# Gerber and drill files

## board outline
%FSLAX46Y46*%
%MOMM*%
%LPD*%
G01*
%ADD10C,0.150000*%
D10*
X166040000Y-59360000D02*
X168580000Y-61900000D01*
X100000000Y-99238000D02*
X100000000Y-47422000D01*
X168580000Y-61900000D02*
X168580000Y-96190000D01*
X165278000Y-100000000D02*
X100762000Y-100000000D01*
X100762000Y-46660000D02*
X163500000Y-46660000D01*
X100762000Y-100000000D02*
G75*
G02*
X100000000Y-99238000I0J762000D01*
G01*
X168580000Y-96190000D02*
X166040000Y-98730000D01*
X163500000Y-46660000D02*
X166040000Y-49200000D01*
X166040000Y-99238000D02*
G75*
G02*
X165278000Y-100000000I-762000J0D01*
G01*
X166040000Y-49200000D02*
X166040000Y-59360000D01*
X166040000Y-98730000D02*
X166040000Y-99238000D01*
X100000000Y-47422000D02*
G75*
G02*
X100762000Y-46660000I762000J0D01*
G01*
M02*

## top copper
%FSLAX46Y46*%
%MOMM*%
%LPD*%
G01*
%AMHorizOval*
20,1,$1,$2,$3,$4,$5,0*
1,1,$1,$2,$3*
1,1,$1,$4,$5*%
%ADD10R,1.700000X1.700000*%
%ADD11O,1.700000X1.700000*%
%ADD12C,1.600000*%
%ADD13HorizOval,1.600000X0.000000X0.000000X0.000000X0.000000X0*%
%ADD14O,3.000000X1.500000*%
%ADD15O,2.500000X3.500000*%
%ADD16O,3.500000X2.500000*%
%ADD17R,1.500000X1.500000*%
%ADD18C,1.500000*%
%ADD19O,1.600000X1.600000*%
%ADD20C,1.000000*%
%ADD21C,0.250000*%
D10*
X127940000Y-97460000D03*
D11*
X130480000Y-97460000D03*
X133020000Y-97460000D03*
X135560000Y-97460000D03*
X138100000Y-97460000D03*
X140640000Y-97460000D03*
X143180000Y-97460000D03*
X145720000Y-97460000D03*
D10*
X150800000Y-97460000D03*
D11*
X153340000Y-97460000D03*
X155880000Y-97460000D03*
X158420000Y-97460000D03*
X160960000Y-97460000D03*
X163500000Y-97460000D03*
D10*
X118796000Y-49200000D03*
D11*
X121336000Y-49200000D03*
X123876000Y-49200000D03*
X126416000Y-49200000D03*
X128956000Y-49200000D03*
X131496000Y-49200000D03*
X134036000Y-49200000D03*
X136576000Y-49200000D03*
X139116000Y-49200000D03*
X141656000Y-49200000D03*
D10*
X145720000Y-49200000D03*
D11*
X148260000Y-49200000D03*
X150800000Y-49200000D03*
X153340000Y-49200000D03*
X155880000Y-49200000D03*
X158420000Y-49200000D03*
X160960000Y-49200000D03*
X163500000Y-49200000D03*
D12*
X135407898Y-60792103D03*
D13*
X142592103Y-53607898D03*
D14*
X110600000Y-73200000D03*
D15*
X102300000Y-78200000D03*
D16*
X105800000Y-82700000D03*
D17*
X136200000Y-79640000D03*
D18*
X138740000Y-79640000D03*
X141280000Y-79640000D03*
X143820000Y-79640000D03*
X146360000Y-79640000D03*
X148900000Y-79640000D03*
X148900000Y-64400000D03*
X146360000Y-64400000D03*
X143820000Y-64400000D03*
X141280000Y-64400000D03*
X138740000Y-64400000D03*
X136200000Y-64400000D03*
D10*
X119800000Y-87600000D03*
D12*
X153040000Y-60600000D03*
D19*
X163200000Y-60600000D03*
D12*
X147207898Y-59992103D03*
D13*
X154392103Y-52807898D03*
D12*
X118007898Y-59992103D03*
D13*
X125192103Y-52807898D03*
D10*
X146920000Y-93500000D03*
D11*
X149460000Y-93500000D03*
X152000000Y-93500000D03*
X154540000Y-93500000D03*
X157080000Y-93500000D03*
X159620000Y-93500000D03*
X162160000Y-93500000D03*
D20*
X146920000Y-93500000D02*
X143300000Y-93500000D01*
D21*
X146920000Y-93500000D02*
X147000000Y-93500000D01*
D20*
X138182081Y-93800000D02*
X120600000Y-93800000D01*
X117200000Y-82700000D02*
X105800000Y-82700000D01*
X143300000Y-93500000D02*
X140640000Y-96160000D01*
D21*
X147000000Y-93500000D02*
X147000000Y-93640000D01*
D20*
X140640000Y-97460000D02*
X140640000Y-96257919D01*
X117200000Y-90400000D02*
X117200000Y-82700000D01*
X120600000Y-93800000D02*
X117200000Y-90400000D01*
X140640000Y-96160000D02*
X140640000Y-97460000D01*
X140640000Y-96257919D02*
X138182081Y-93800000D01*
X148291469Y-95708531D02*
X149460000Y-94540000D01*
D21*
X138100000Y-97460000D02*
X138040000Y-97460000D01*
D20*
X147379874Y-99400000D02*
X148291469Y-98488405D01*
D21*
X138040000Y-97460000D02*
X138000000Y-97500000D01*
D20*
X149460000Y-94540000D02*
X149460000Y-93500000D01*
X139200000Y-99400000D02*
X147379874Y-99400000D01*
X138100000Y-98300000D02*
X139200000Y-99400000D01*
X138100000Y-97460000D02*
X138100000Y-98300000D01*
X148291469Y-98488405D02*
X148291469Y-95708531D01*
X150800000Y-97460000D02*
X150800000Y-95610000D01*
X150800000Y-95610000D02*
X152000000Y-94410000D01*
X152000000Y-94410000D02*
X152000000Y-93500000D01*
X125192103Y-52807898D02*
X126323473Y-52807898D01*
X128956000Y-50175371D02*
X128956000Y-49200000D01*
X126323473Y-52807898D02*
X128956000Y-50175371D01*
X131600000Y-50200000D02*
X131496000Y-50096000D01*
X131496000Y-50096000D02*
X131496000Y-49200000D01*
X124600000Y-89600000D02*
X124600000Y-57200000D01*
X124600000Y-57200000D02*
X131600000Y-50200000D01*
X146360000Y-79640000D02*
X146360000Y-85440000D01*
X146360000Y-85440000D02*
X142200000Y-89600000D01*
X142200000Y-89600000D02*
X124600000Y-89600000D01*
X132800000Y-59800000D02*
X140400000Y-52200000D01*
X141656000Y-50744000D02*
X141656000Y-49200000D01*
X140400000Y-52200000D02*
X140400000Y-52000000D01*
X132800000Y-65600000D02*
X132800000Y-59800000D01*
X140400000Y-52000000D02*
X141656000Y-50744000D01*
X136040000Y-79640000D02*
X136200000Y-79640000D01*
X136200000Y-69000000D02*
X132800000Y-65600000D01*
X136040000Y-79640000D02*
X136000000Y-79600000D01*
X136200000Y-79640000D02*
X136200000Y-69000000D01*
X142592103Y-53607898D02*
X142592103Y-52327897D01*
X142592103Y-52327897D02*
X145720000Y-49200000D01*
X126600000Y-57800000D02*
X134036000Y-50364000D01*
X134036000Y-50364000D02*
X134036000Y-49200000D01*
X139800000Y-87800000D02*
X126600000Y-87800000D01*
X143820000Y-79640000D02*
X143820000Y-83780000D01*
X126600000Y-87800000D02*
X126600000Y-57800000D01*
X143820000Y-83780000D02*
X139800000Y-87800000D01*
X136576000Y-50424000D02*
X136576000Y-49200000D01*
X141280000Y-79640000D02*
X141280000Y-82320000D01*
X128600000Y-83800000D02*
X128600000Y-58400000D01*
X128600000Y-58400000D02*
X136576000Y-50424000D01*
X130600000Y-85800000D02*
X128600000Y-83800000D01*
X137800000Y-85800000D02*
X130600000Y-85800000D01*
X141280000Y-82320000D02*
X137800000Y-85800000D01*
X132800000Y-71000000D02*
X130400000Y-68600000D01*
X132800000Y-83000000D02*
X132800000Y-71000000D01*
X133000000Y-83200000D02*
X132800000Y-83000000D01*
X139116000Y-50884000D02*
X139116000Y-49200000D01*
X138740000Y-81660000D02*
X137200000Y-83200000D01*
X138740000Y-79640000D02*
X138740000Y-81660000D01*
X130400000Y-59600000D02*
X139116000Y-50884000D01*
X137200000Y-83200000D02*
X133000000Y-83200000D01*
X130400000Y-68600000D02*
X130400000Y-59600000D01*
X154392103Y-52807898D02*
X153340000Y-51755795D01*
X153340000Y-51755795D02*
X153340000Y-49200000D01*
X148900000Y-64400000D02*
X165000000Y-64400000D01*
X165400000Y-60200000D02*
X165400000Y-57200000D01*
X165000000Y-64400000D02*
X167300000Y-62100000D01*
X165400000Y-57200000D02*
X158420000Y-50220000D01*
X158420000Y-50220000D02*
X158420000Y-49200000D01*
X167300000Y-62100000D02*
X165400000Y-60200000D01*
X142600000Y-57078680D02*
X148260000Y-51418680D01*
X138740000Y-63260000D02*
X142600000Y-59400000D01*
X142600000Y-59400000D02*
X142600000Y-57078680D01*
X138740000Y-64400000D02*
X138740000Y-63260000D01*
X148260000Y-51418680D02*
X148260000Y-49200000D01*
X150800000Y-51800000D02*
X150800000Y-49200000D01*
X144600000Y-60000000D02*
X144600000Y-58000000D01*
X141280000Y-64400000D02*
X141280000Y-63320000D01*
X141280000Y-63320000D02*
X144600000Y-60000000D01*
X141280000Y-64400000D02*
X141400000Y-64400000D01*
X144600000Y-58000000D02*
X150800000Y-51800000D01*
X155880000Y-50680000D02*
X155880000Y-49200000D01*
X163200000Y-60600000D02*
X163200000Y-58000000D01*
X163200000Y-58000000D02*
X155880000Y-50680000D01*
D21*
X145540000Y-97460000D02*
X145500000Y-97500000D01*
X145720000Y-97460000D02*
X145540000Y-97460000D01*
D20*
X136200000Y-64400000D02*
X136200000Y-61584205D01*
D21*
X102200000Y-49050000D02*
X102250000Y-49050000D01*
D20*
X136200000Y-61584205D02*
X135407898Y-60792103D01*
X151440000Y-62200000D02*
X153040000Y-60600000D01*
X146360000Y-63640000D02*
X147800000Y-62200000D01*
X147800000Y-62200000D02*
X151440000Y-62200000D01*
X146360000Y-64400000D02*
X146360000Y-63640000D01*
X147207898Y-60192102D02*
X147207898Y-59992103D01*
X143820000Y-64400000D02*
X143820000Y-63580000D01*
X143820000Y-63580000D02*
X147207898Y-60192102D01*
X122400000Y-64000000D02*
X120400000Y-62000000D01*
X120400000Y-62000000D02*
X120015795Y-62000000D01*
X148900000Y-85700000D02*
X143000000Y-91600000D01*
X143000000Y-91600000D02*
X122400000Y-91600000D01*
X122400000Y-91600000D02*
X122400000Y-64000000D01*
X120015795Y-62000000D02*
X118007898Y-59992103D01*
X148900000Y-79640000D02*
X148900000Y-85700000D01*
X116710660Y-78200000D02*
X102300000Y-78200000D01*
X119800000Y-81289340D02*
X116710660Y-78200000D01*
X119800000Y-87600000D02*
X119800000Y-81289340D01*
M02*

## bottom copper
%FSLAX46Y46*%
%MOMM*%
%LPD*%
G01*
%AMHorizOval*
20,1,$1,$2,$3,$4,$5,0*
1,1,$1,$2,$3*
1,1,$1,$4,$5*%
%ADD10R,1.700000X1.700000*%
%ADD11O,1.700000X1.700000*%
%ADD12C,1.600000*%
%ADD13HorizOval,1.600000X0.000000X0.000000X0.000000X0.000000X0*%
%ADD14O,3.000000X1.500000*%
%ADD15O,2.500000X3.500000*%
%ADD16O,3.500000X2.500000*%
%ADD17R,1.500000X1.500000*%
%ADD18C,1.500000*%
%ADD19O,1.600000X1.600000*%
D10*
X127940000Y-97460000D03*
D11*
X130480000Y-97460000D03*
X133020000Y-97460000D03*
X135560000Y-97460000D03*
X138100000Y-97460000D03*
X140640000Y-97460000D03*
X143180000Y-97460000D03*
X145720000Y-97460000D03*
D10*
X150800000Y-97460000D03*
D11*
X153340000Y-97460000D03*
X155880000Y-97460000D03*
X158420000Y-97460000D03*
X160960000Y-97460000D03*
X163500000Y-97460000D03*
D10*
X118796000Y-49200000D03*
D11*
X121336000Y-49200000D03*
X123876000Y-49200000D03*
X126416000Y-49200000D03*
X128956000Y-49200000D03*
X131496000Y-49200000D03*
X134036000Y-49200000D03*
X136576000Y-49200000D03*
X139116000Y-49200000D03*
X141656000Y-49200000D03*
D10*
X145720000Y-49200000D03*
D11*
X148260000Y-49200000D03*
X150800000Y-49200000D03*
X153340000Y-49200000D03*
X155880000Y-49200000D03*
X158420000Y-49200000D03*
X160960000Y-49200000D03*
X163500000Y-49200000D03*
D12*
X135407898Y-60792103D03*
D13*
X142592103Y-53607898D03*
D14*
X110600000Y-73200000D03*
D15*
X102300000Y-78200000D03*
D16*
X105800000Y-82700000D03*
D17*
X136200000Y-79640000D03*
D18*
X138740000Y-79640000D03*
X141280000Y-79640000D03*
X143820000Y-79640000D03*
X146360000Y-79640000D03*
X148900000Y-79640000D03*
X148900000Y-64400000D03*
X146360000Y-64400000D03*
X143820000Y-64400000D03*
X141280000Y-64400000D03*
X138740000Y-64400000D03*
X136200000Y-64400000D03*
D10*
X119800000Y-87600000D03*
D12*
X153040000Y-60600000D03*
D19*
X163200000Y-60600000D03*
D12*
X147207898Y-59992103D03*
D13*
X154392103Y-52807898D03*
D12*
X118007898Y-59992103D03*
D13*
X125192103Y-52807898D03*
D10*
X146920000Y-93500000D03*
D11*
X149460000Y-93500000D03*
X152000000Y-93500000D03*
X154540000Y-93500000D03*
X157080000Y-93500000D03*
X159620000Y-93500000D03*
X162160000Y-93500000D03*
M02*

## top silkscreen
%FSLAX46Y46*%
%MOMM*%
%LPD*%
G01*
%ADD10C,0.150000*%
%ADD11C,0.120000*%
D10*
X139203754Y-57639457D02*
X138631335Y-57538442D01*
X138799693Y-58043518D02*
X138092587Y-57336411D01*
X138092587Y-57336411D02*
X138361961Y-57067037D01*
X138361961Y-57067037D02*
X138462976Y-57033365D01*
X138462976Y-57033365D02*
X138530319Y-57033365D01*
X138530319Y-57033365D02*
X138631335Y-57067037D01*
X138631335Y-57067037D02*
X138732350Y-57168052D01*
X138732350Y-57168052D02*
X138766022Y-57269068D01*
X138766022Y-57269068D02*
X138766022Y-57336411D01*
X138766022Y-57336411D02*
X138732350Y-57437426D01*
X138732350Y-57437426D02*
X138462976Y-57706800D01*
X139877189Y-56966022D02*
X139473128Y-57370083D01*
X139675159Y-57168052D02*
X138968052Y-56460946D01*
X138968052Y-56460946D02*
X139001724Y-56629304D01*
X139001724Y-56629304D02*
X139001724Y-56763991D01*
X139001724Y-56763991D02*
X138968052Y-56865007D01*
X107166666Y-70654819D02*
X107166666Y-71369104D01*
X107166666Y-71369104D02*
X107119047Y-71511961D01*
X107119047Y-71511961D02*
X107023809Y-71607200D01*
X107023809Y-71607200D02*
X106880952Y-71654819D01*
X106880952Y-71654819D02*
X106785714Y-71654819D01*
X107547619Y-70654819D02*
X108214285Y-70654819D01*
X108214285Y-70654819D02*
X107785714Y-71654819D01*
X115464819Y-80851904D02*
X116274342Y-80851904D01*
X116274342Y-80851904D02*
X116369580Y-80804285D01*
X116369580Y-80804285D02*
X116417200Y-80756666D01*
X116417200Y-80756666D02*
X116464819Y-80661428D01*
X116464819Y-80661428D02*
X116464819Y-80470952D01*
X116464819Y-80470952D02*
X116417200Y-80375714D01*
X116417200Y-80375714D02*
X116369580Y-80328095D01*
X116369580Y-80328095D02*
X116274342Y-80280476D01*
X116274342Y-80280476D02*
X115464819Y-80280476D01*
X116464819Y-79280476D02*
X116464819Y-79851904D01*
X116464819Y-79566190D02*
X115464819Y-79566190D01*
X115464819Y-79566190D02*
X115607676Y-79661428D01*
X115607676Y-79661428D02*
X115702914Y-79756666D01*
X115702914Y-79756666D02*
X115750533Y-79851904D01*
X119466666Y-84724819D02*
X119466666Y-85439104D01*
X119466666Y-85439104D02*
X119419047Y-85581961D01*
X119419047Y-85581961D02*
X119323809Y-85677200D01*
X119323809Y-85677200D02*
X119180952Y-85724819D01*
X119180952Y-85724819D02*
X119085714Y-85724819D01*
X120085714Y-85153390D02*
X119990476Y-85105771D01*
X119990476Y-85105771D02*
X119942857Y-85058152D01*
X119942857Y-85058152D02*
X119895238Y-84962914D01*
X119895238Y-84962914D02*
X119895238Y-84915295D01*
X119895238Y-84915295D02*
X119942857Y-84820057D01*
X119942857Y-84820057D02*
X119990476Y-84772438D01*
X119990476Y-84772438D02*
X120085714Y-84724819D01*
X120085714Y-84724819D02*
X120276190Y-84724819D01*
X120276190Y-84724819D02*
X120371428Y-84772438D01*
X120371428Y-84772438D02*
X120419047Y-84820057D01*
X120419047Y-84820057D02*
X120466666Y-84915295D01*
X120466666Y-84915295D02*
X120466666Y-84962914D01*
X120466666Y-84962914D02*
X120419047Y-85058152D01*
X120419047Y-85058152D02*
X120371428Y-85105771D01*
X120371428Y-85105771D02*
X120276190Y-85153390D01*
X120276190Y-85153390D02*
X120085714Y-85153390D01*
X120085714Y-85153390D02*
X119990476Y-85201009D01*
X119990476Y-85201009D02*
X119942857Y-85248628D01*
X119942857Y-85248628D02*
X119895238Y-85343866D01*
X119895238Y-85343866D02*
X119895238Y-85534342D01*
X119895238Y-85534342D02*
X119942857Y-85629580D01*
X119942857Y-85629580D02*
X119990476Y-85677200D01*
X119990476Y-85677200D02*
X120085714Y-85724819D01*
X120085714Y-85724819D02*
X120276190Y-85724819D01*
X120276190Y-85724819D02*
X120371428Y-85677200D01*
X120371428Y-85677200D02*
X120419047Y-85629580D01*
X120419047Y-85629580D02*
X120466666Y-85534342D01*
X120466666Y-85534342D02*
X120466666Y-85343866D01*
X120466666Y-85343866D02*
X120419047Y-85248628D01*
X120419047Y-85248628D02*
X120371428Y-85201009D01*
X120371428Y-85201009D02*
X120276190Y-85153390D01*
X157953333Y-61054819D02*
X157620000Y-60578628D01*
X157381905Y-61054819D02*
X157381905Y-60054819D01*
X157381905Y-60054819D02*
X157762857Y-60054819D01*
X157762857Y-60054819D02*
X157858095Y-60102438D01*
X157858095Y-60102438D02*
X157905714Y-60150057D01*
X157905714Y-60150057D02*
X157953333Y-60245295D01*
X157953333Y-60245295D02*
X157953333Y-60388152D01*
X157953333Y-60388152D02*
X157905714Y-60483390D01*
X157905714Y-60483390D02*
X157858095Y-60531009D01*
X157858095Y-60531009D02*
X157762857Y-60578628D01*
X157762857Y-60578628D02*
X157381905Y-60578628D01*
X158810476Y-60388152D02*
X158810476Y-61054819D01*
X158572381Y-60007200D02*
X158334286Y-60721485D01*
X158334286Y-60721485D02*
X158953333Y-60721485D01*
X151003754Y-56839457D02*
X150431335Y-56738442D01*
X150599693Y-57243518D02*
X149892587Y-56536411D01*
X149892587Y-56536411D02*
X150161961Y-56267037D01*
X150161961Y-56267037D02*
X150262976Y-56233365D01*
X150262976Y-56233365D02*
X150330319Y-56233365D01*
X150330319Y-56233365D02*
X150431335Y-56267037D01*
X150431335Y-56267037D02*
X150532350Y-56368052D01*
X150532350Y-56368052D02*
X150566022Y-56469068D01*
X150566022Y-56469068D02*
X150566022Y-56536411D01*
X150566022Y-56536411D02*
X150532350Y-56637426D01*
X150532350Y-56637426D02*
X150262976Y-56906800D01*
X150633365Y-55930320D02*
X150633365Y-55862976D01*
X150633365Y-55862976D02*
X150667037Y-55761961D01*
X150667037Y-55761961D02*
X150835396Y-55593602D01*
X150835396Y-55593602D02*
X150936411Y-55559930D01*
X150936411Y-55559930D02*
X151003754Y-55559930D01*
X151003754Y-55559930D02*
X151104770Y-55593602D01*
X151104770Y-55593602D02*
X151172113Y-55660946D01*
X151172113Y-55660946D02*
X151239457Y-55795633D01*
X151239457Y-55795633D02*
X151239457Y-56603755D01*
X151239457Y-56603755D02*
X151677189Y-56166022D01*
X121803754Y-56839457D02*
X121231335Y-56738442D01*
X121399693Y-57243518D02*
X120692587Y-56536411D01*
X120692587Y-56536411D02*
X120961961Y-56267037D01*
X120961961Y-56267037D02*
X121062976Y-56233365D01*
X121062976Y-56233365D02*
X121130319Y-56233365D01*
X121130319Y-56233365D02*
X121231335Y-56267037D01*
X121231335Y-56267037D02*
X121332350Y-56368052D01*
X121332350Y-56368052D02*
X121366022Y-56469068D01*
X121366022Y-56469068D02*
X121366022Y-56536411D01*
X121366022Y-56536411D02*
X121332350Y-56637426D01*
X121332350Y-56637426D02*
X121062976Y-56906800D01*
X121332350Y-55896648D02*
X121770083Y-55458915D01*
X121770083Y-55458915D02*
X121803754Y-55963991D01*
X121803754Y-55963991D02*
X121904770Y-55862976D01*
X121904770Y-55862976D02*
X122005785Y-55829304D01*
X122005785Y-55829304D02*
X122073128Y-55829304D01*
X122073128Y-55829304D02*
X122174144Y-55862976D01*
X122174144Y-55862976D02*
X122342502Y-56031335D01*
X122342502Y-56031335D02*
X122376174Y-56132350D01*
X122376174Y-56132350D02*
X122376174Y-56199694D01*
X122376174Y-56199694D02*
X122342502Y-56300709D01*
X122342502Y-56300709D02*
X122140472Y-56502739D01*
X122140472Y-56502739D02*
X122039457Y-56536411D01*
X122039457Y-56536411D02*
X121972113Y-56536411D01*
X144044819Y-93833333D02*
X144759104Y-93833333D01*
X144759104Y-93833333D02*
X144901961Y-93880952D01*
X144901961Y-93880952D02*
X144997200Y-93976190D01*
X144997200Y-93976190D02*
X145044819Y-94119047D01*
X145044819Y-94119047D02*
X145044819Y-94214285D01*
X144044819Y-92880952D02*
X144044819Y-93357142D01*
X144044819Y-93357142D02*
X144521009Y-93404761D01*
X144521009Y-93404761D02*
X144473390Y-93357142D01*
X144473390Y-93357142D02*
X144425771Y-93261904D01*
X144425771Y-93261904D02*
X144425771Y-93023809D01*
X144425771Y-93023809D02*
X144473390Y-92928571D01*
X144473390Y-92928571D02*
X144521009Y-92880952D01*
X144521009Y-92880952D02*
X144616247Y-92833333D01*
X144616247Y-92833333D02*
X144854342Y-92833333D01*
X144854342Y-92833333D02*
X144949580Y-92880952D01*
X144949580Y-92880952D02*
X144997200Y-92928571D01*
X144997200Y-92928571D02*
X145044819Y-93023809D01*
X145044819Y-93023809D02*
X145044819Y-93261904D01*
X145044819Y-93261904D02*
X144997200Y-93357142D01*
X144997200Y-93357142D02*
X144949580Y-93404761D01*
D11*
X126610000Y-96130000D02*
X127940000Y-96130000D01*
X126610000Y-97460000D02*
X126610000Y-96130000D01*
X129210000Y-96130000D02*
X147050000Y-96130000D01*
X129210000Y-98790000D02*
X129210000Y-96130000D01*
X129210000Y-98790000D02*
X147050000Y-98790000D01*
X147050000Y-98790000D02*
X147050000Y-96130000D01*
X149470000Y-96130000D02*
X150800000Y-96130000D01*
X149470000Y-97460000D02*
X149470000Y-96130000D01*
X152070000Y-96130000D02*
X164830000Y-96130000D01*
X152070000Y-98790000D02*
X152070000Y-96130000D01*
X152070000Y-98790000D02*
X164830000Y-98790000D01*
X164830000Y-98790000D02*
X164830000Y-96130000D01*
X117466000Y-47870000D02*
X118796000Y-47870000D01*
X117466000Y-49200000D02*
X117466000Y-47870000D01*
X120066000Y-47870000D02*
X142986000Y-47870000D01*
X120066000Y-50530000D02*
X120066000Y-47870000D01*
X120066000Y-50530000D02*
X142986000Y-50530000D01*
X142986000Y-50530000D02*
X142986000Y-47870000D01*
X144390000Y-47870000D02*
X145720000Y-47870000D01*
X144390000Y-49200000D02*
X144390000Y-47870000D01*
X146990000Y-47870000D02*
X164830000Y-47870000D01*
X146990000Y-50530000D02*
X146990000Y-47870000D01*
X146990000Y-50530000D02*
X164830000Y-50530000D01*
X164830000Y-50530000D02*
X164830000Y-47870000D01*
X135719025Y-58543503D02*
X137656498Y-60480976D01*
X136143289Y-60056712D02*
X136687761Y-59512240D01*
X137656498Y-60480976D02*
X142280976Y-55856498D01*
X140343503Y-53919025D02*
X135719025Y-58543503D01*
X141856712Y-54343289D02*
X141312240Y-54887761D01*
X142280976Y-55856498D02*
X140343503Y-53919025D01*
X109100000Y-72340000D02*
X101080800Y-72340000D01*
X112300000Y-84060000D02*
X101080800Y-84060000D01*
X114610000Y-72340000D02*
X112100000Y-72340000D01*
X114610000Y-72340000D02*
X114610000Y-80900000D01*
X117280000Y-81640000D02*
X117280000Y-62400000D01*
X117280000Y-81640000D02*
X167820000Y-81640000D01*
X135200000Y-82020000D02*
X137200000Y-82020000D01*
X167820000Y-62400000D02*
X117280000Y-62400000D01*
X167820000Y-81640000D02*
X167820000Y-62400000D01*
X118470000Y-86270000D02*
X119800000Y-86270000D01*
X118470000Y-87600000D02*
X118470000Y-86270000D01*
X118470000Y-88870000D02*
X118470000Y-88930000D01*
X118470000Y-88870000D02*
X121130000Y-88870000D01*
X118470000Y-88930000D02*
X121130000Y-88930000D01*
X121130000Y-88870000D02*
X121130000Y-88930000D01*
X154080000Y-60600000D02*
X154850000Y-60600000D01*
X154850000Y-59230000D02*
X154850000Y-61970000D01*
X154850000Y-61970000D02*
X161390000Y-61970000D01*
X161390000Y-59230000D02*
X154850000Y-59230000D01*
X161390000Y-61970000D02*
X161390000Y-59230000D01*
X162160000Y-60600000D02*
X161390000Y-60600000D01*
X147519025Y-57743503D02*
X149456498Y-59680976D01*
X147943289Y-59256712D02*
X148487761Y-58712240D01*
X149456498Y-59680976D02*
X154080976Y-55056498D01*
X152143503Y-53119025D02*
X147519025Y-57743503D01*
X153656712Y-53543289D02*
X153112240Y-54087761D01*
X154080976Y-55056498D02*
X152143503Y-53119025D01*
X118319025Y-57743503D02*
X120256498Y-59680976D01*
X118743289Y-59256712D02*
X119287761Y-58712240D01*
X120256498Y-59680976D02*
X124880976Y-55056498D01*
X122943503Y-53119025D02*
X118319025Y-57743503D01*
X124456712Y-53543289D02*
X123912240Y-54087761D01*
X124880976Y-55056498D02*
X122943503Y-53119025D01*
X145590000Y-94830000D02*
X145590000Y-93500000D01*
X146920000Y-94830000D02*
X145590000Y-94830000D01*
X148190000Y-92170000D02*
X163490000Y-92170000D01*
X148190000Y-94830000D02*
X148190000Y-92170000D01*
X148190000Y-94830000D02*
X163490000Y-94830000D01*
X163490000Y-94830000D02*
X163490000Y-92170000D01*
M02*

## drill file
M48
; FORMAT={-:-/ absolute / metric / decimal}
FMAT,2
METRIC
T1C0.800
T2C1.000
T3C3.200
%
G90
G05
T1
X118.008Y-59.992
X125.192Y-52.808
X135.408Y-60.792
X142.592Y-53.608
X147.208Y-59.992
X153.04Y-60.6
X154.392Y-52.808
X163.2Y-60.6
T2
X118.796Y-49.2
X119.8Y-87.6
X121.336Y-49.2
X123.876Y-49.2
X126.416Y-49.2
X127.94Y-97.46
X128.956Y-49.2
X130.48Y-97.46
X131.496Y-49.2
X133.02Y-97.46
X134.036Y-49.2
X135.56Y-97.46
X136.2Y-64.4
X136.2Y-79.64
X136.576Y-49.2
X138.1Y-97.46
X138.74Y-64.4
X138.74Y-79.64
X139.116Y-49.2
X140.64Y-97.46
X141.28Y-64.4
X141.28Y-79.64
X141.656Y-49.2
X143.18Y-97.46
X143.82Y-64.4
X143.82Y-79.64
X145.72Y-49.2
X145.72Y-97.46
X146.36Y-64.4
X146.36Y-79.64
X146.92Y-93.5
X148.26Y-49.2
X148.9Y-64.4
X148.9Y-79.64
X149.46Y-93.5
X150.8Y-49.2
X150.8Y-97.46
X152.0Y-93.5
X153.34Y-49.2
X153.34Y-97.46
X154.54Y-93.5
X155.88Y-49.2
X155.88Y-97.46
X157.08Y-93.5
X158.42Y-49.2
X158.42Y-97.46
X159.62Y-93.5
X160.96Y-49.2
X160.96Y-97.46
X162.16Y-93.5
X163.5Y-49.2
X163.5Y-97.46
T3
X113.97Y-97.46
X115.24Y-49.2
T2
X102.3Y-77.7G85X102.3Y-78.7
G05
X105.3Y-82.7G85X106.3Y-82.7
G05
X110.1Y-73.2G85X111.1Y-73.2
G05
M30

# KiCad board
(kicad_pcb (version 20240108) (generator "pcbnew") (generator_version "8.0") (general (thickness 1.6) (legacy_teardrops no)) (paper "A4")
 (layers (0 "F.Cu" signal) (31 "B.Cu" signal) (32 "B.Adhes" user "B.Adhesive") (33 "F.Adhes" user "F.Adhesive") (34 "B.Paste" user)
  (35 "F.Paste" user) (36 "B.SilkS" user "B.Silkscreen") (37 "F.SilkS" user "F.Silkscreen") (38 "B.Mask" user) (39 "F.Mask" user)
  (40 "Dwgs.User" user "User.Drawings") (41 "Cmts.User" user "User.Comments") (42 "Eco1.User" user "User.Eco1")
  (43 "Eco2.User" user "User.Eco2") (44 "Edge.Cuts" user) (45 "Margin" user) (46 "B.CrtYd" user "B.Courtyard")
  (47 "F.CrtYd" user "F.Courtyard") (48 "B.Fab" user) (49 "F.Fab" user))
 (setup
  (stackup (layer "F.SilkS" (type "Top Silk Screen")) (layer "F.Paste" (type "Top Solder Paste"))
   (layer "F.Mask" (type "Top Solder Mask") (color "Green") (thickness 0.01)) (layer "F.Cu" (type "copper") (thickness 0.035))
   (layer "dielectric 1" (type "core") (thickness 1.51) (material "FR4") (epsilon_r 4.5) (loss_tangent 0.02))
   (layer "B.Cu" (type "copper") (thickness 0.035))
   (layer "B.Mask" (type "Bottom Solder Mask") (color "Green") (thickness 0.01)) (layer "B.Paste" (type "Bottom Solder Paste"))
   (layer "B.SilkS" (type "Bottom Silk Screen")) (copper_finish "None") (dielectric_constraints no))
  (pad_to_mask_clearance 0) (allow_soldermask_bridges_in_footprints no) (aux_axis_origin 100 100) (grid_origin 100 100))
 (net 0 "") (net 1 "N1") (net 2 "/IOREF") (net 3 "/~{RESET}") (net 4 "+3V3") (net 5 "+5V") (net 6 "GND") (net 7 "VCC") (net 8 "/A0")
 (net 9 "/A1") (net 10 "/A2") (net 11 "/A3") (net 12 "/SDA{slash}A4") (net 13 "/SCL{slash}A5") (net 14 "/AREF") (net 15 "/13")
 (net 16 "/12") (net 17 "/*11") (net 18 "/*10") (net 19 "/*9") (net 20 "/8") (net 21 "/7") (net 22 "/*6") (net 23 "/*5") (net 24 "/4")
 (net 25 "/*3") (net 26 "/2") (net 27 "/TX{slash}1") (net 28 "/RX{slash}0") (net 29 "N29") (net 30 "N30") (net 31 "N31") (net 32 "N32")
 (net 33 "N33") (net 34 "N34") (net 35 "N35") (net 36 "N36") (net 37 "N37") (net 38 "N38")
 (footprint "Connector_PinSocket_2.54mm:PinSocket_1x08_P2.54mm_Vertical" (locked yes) (layer "F.Cu") (at 127.94 97.46 90)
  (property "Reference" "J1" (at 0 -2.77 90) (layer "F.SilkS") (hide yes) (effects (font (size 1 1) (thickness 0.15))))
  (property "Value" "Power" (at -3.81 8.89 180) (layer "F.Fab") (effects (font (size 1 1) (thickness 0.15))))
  (fp_line (start 1.33 -1.33) (end 1.33 0) (stroke (width 0.12) (type solid)) (layer "F.SilkS"))
  (fp_line (start 0 -1.33) (end 1.33 -1.33) (stroke (width 0.12) (type solid)) (layer "F.SilkS"))
  (fp_line (start 1.33 1.27) (end 1.33 19.11) (stroke (width 0.12) (type solid)) (layer "F.SilkS"))
  (fp_line (start -1.33 1.27) (end 1.33 1.27) (stroke (width 0.12) (type solid)) (layer "F.SilkS"))
  (fp_line (start -1.33 1.27) (end -1.33 19.11) (stroke (width 0.12) (type solid)) (layer "F.SilkS"))
  (fp_line (start -1.33 19.11) (end 1.33 19.11) (stroke (width 0.12) (type solid)) (layer "F.SilkS"))
  (pad "1" thru_hole rect (at 0 0 90) (size 1.7 1.7) (drill 1) (layers "*.Cu" "*.Mask") (remove_unused_layers no) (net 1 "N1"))
  (pad "2" thru_hole oval (at 0 2.54 90) (size 1.7 1.7) (drill 1) (layers "*.Cu" "*.Mask") (remove_unused_layers no) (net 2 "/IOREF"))
  (pad "3" thru_hole oval (at 0 5.08 90) (size 1.7 1.7) (drill 1) (layers "*.Cu" "*.Mask") (remove_unused_layers no) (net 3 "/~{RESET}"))
  (pad "4" thru_hole oval (at 0 7.62 90) (size 1.7 1.7) (drill 1) (layers "*.Cu" "*.Mask") (remove_unused_layers no) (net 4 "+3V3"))
  (pad "5" thru_hole oval (at 0 10.16 90) (size 1.7 1.7) (drill 1) (layers "*.Cu" "*.Mask") (remove_unused_layers no) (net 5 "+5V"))
  (pad "6" thru_hole oval (at 0 12.7 90) (size 1.7 1.7) (drill 1) (layers "*.Cu" "*.Mask") (remove_unused_layers no) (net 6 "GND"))
  (pad "7" thru_hole oval (at 0 15.24 90) (size 1.7 1.7) (drill 1) (layers "*.Cu" "*.Mask") (remove_unused_layers no) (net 6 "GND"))
  (pad "8" thru_hole oval (at 0 17.78 90) (size 1.7 1.7) (drill 1) (layers "*.Cu" "*.Mask") (remove_unused_layers no) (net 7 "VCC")))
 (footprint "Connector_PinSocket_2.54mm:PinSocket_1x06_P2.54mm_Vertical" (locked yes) (layer "F.Cu") (at 150.8 97.46 90)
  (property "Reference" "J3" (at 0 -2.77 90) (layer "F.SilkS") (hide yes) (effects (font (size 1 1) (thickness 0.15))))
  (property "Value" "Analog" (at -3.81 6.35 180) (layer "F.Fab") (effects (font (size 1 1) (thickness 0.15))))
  (fp_line (start 1.33 -1.33) (end 1.33 0) (stroke (width 0.12) (type solid)) (layer "F.SilkS"))
  (fp_line (start 0 -1.33) (end 1.33 -1.33) (stroke (width 0.12) (type solid)) (layer "F.SilkS"))
  (fp_line (start 1.33 1.27) (end 1.33 14.03) (stroke (width 0.12) (type solid)) (layer "F.SilkS"))
  (fp_line (start -1.33 1.27) (end 1.33 1.27) (stroke (width 0.12) (type solid)) (layer "F.SilkS"))
  (fp_line (start -1.33 1.27) (end -1.33 14.03) (stroke (width 0.12) (type solid)) (layer "F.SilkS"))
  (fp_line (start -1.33 14.03) (end 1.33 14.03) (stroke (width 0.12) (type solid)) (layer "F.SilkS"))
  (pad "1" thru_hole rect (at 0 0 90) (size 1.7 1.7) (drill 1) (layers "*.Cu" "*.Mask") (remove_unused_layers no) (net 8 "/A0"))
  (pad "2" thru_hole oval (at 0 2.54 90) (size 1.7 1.7) (drill 1) (layers "*.Cu" "*.Mask") (remove_unused_layers no) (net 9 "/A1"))
  (pad "3" thru_hole oval (at 0 5.08 90) (size 1.7 1.7) (drill 1) (layers "*.Cu" "*.Mask") (remove_unused_layers no) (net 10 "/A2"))
  (pad "4" thru_hole oval (at 0 7.62 90) (size 1.7 1.7) (drill 1) (layers "*.Cu" "*.Mask") (remove_unused_layers no) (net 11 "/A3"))
  (pad "5" thru_hole oval (at 0 10.16 90) (size 1.7 1.7) (drill 1) (layers "*.Cu" "*.Mask") (remove_unused_layers no)
   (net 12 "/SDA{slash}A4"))
  (pad "6" thru_hole oval (at 0 12.7 90) (size 1.7 1.7) (drill 1) (layers "*.Cu" "*.Mask") (remove_unused_layers no)
   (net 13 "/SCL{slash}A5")))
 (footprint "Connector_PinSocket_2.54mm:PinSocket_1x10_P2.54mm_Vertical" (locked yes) (layer "F.Cu") (at 118.796 49.2 90)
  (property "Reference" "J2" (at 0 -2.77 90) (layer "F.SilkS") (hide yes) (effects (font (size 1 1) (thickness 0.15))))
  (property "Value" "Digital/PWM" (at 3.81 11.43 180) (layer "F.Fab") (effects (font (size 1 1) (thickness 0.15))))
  (fp_line (start 1.33 -1.33) (end 1.33 0) (stroke (width 0.12) (type solid)) (layer "F.SilkS"))
  (fp_line (start 0 -1.33) (end 1.33 -1.33) (stroke (width 0.12) (type solid)) (layer "F.SilkS"))
  (fp_line (start 1.33 1.27) (end 1.33 24.19) (stroke (width 0.12) (type solid)) (layer "F.SilkS"))
  (fp_line (start -1.33 1.27) (end 1.33 1.27) (stroke (width 0.12) (type solid)) (layer "F.SilkS"))
  (fp_line (start -1.33 1.27) (end -1.33 24.19) (stroke (width 0.12) (type solid)) (layer "F.SilkS"))
  (fp_line (start -1.33 24.19) (end 1.33 24.19) (stroke (width 0.12) (type solid)) (layer "F.SilkS"))
  (pad "1" thru_hole rect (at 0 0 90) (size 1.7 1.7) (drill 1) (layers "*.Cu" "*.Mask") (remove_unused_layers no) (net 13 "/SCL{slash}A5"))
  (pad "2" thru_hole oval (at 0 2.54 90) (size 1.7 1.7) (drill 1) (layers "*.Cu" "*.Mask") (remove_unused_layers no)
   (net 12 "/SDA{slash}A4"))
  (pad "3" thru_hole oval (at 0 5.08 90) (size 1.7 1.7) (drill 1) (layers "*.Cu" "*.Mask") (remove_unused_layers no) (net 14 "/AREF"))
  (pad "4" thru_hole oval (at 0 7.62 90) (size 1.7 1.7) (drill 1) (layers "*.Cu" "*.Mask") (remove_unused_layers no) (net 6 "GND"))
  (pad "5" thru_hole oval (at 0 10.16 90) (size 1.7 1.7) (drill 1) (layers "*.Cu" "*.Mask") (remove_unused_layers no) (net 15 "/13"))
  (pad "6" thru_hole oval (at 0 12.7 90) (size 1.7 1.7) (drill 1) (layers "*.Cu" "*.Mask") (remove_unused_layers no) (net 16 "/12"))
  (pad "7" thru_hole oval (at 0 15.24 90) (size 1.7 1.7) (drill 1) (layers "*.Cu" "*.Mask") (remove_unused_layers no) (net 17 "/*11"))
  (pad "8" thru_hole oval (at 0 17.78 90) (size 1.7 1.7) (drill 1) (layers "*.Cu" "*.Mask") (remove_unused_layers no) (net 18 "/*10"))
  (pad "9" thru_hole oval (at 0 20.32 90) (size 1.7 1.7) (drill 1) (layers "*.Cu" "*.Mask") (remove_unused_layers no) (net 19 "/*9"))
  (pad "10" thru_hole oval (at 0 22.86 90) (size 1.7 1.7) (drill 1) (layers "*.Cu" "*.Mask") (remove_unused_layers no) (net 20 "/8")))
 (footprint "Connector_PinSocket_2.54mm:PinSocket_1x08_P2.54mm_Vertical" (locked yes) (layer "F.Cu") (at 145.72 49.2 90)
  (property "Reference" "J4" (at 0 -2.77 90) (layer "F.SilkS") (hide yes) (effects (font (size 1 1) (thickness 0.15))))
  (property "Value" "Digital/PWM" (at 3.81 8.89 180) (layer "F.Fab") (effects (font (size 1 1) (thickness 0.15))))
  (fp_line (start 1.33 -1.33) (end 1.33 0) (stroke (width 0.12) (type solid)) (layer "F.SilkS"))
  (fp_line (start 0 -1.33) (end 1.33 -1.33) (stroke (width 0.12) (type solid)) (layer "F.SilkS"))
  (fp_line (start 1.33 1.27) (end 1.33 19.11) (stroke (width 0.12) (type solid)) (layer "F.SilkS"))
  (fp_line (start -1.33 1.27) (end 1.33 1.27) (stroke (width 0.12) (type solid)) (layer "F.SilkS"))
  (fp_line (start -1.33 1.27) (end -1.33 19.11) (stroke (width 0.12) (type solid)) (layer "F.SilkS"))
  (fp_line (start -1.33 19.11) (end 1.33 19.11) (stroke (width 0.12) (type solid)) (layer "F.SilkS"))
  (pad "1" thru_hole rect (at 0 0 90) (size 1.7 1.7) (drill 1) (layers "*.Cu" "*.Mask") (remove_unused_layers no) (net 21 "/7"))
  (pad "2" thru_hole oval (at 0 2.54 90) (size 1.7 1.7) (drill 1) (layers "*.Cu" "*.Mask") (remove_unused_layers no) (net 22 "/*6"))
  (pad "3" thru_hole oval (at 0 5.08 90) (size 1.7 1.7) (drill 1) (layers "*.Cu" "*.Mask") (remove_unused_layers no) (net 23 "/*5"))
  (pad "4" thru_hole oval (at 0 7.62 90) (size 1.7 1.7) (drill 1) (layers "*.Cu" "*.Mask") (remove_unused_layers no) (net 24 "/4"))
  (pad "5" thru_hole oval (at 0 10.16 90) (size 1.7 1.7) (drill 1) (layers "*.Cu" "*.Mask") (remove_unused_layers no) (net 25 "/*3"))
  (pad "6" thru_hole oval (at 0 12.7 90) (size 1.7 1.7) (drill 1) (layers "*.Cu" "*.Mask") (remove_unused_layers no) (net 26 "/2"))
  (pad "7" thru_hole oval (at 0 15.24 90) (size 1.7 1.7) (drill 1) (layers "*.Cu" "*.Mask") (remove_unused_layers no) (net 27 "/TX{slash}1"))
  (pad "8" thru_hole oval (at 0 17.78 90) (size 1.7 1.7) (drill 1) (layers "*.Cu" "*.Mask") (remove_unused_layers no) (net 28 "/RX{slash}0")))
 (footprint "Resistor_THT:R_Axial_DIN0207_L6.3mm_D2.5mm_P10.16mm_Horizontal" (layer "F.Cu") (at 135.407898 60.792103 45)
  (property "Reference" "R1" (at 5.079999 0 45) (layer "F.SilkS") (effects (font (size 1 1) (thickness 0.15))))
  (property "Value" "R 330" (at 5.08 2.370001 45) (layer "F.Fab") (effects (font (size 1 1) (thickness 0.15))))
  (fp_line (start 1.81 -1.37) (end 1.81 1.37) (stroke (width 0.12) (type solid)) (layer "F.SilkS"))
  (fp_line (start 1.04 0) (end 1.81 0) (stroke (width 0.12) (type solid)) (layer "F.SilkS"))
  (fp_line (start 1.81 1.37) (end 8.35 1.37) (stroke (width 0.12) (type solid)) (layer "F.SilkS"))
  (fp_line (start 8.35 -1.37) (end 1.81 -1.37) (stroke (width 0.12) (type solid)) (layer "F.SilkS"))
  (fp_line (start 9.12 0) (end 8.350001 0) (stroke (width 0.12) (type solid)) (layer "F.SilkS"))
  (fp_line (start 8.35 1.37) (end 8.35 -1.37) (stroke (width 0.12) (type solid)) (layer "F.SilkS"))
  (pad "1" thru_hole circle (at 0 0 45) (size 1.6 1.6) (drill 0.8) (layers "*.Cu" "*.Mask") (remove_unused_layers no) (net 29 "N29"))
  (pad "2" thru_hole oval (at 10.16 0 45) (size 1.6 1.6) (drill 0.8) (layers "*.Cu" "*.Mask") (remove_unused_layers no) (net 21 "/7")))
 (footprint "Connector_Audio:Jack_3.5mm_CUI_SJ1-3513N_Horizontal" (layer "F.Cu") (at 102.3 78.2)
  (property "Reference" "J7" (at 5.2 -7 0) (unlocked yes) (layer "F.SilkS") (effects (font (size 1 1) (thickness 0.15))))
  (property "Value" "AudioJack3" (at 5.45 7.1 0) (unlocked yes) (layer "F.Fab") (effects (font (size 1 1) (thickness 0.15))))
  (fp_line (start 6.8 -5.86) (end -1.2192 -5.86) (stroke (width 0.12) (type solid)) (layer "F.SilkS"))
  (fp_line (start 10 5.86) (end -1.2192 5.86) (stroke (width 0.12) (type solid)) (layer "F.SilkS"))
  (fp_line (start 12.31 -5.86) (end 9.8 -5.86) (stroke (width 0.12) (type solid)) (layer "F.SilkS"))
  (fp_line (start 12.31 -5.86) (end 12.31 2.7) (stroke (width 0.12) (type solid)) (layer "F.SilkS"))
  (pad "R" thru_hole oval (at 8.3 -5) (size 3 1.5) (drill oval 2 1) (layers "*.Cu" "*.Mask") (remove_unused_layers no) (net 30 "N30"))
  (pad "S" thru_hole oval (at 0 0 270) (size 3.5 2.5) (drill oval 2 1) (layers "*.Cu" "*.Mask") (remove_unused_layers no) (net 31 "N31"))
  (pad "T" thru_hole oval (at 3.5 4.5) (size 3.5 2.5) (drill oval 2 1) (layers "*.Cu" "*.Mask") (remove_unused_layers no) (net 6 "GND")))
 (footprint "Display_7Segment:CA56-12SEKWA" (layer "F.Cu") (at 136.2 79.64 90)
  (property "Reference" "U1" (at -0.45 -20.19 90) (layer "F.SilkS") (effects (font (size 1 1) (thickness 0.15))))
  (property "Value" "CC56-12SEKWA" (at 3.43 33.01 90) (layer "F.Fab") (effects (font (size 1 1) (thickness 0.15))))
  (fp_line (start -2 -18.92) (end 17.24 -18.92) (stroke (width 0.12) (type solid)) (layer "F.SilkS"))
  (fp_line (start -2 -18.92) (end -2 31.62) (stroke (width 0.12) (type solid)) (layer "F.SilkS"))
  (fp_line (start -2.38 -1) (end -2.38 1) (stroke (width 0.12) (type solid)) (layer "F.SilkS"))
  (fp_line (start 17.24 31.62) (end 17.24 -18.92) (stroke (width 0.12) (type solid)) (layer "F.SilkS"))
  (fp_line (start -2 31.62) (end 17.24 31.62) (stroke (width 0.12) (type solid)) (layer "F.SilkS"))
  (pad "1" thru_hole rect (at 0 0 90) (size 1.5 1.5) (drill 1) (layers "*.Cu" "*.Mask") (remove_unused_layers no) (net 20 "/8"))
  (pad "2" thru_hole circle (at 0 2.54 90) (size 1.5 1.5) (drill 1) (layers "*.Cu" "*.Mask") (remove_unused_layers no) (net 19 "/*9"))
  (pad "3" thru_hole circle (at 0 5.08 90) (size 1.5 1.5) (drill 1) (layers "*.Cu" "*.Mask") (remove_unused_layers no) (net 18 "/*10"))
  (pad "4" thru_hole circle (at 0 7.62 90) (size 1.5 1.5) (drill 1) (layers "*.Cu" "*.Mask") (remove_unused_layers no) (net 17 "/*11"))
  (pad "5" thru_hole circle (at 0 10.16 90) (size 1.5 1.5) (drill 1) (layers "*.Cu" "*.Mask") (remove_unused_layers no) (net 16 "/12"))
  (pad "6" thru_hole circle (at 0 12.7 90) (size 1.5 1.5) (drill 1) (layers "*.Cu" "*.Mask") (remove_unused_layers no) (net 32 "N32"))
  (pad "7" thru_hole circle (at 15.24 12.7 90) (size 1.5 1.5) (drill 1) (layers "*.Cu" "*.Mask") (remove_unused_layers no) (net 26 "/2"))
  (pad "8" thru_hole circle (at 15.24 10.16 90) (size 1.5 1.5) (drill 1) (layers "*.Cu" "*.Mask") (remove_unused_layers no) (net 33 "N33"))
  (pad "9" thru_hole circle (at 15.24 7.62 90) (size 1.5 1.5) (drill 1) (layers "*.Cu" "*.Mask") (remove_unused_layers no) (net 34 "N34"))
  (pad "10" thru_hole circle (at 15.24 5.08 90) (size 1.5 1.5) (drill 1) (layers "*.Cu" "*.Mask") (remove_unused_layers no) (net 23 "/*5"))
  (pad "11" thru_hole circle (at 15.24 2.54 90) (size 1.5 1.5) (drill 1) (layers "*.Cu" "*.Mask") (remove_unused_layers no) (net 22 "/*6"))
  (pad "12" thru_hole circle (at 15.24 0 90) (size 1.5 1.5) (drill 1) (layers "*.Cu" "*.Mask") (remove_unused_layers no) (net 29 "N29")))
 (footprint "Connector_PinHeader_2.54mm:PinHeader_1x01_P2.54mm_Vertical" (layer "F.Cu") (at 119.8 87.6)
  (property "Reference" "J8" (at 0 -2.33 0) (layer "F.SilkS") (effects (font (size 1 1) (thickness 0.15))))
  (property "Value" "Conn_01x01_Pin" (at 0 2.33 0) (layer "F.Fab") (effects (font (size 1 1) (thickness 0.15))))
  (fp_line (start -1.33 -1.33) (end 0 -1.33) (stroke (width 0.12) (type solid)) (layer "F.SilkS"))
  (fp_line (start -1.33 0) (end -1.33 -1.33) (stroke (width 0.12) (type solid)) (layer "F.SilkS"))
  (fp_line (start -1.33 1.27) (end -1.33 1.33) (stroke (width 0.12) (type solid)) (layer "F.SilkS"))
  (fp_line (start -1.33 1.27) (end 1.33 1.27) (stroke (width 0.12) (type solid)) (layer "F.SilkS"))
  (fp_line (start -1.33 1.33) (end 1.33 1.33) (stroke (width 0.12) (type solid)) (layer "F.SilkS"))
  (fp_line (start 1.33 1.27) (end 1.33 1.33) (stroke (width 0.12) (type solid)) (layer "F.SilkS"))
  (pad "1" thru_hole rect (at 0 0) (size 1.7 1.7) (drill 1) (layers "*.Cu" "*.Mask") (remove_unused_layers no) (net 31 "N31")))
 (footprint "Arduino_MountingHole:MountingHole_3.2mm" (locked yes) (layer "F.Cu") (at 115.24 49.2)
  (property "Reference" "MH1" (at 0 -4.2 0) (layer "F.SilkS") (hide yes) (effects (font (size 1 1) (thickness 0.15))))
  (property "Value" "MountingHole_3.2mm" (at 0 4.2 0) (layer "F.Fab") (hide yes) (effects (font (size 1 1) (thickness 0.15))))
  (pad "" np_thru_hole circle (at 0 0) (size 3.2 3.2) (drill 3.2) (layers "*.Cu" "*.Mask")))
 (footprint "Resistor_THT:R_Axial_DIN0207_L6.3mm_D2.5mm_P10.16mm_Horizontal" (layer "F.Cu") (at 153.04 60.6)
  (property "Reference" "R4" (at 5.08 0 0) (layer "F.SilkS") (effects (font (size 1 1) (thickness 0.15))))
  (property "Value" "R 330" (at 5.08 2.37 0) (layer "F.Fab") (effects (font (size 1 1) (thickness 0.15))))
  (fp_line (start 1.04 0) (end 1.81 0) (stroke (width 0.12) (type solid)) (layer "F.SilkS"))
  (fp_line (start 1.81 -1.37) (end 1.81 1.37) (stroke (width 0.12) (type solid)) (layer "F.SilkS"))
  (fp_line (start 1.81 1.37) (end 8.35 1.37) (stroke (width 0.12) (type solid)) (layer "F.SilkS"))
  (fp_line (start 8.35 -1.37) (end 1.81 -1.37) (stroke (width 0.12) (type solid)) (layer "F.SilkS"))
  (fp_line (start 8.35 1.37) (end 8.35 -1.37) (stroke (width 0.12) (type solid)) (layer "F.SilkS"))
  (fp_line (start 9.12 0) (end 8.35 0) (stroke (width 0.12) (type solid)) (layer "F.SilkS"))
  (pad "1" thru_hole circle (at 0 0) (size 1.6 1.6) (drill 0.8) (layers "*.Cu" "*.Mask") (remove_unused_layers no) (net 33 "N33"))
  (pad "2" thru_hole oval (at 10.16 0) (size 1.6 1.6) (drill 0.8) (layers "*.Cu" "*.Mask") (remove_unused_layers no) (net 25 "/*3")))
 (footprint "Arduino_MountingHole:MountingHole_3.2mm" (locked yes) (layer "F.Cu") (at 113.97 97.46)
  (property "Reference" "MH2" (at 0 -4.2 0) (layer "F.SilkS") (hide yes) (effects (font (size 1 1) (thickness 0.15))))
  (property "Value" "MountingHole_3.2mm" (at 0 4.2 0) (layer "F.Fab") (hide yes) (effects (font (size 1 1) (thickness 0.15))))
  (pad "" np_thru_hole circle (at 0 0) (size 3.2 3.2) (drill 3.2) (layers "*.Cu" "*.Mask")))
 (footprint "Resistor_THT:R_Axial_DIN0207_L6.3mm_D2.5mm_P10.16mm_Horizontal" (layer "F.Cu") (at 147.207898 59.992103 45)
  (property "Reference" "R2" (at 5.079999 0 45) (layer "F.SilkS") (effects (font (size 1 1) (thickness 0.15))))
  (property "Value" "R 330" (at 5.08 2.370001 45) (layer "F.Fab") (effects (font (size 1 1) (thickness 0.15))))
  (fp_line (start 1.81 -1.37) (end 1.81 1.37) (stroke (width 0.12) (type solid)) (layer "F.SilkS"))
  (fp_line (start 1.04 0) (end 1.81 0) (stroke (width 0.12) (type solid)) (layer "F.SilkS"))
  (fp_line (start 1.81 1.37) (end 8.35 1.37) (stroke (width 0.12) (type solid)) (layer "F.SilkS"))
  (fp_line (start 8.35 -1.37) (end 1.81 -1.37) (stroke (width 0.12) (type solid)) (layer "F.SilkS"))
  (fp_line (start 9.12 0) (end 8.350001 0) (stroke (width 0.12) (type solid)) (layer "F.SilkS"))
  (fp_line (start 8.35 1.37) (end 8.35 -1.37) (stroke (width 0.12) (type solid)) (layer "F.SilkS"))
  (pad "1" thru_hole circle (at 0 0 45) (size 1.6 1.6) (drill 0.8) (layers "*.Cu" "*.Mask") (remove_unused_layers no) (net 34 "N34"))
  (pad "2" thru_hole oval (at 10.16 0 45) (size 1.6 1.6) (drill 0.8) (layers "*.Cu" "*.Mask") (remove_unused_layers no) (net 24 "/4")))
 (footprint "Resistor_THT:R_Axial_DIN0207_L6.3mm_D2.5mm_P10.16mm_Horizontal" (layer "F.Cu") (at 118.007898 59.992103 45)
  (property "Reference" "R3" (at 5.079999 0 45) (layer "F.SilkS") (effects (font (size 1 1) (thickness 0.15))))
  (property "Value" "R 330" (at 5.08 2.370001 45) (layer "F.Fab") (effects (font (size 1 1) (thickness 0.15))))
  (fp_line (start 1.81 -1.37) (end 1.81 1.37) (stroke (width 0.12) (type solid)) (layer "F.SilkS"))
  (fp_line (start 1.04 0) (end 1.81 0) (stroke (width 0.12) (type solid)) (layer "F.SilkS"))
  (fp_line (start 1.81 1.37) (end 8.35 1.37) (stroke (width 0.12) (type solid)) (layer "F.SilkS"))
  (fp_line (start 8.35 -1.37) (end 1.81 -1.37) (stroke (width 0.12) (type solid)) (layer "F.SilkS"))
  (fp_line (start 9.12 0) (end 8.350001 0) (stroke (width 0.12) (type solid)) (layer "F.SilkS"))
  (fp_line (start 8.35 1.37) (end 8.35 -1.37) (stroke (width 0.12) (type solid)) (layer "F.SilkS"))
  (pad "1" thru_hole circle (at 0 0 45) (size 1.6 1.6) (drill 0.8) (layers "*.Cu" "*.Mask") (remove_unused_layers no) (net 32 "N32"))
  (pad "2" thru_hole oval (at 10.16 0 45) (size 1.6 1.6) (drill 0.8) (layers "*.Cu" "*.Mask") (remove_unused_layers no) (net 15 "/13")))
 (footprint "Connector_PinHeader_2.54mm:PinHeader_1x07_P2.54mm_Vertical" (layer "F.Cu") (at 146.92 93.5 90)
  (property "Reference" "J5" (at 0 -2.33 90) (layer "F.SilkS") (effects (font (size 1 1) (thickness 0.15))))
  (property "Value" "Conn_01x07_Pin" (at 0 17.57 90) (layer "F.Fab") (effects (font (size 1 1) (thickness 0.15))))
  (fp_line (start -1.33 -1.33) (end 0 -1.33) (stroke (width 0.12) (type solid)) (layer "F.SilkS"))
  (fp_line (start -1.33 0) (end -1.33 -1.33) (stroke (width 0.12) (type solid)) (layer "F.SilkS"))
  (fp_line (start 1.33 1.27) (end 1.33 16.57) (stroke (width 0.12) (type solid)) (layer "F.SilkS"))
  (fp_line (start -1.33 1.27) (end 1.33 1.27) (stroke (width 0.12) (type solid)) (layer "F.SilkS"))
  (fp_line (start -1.33 1.27) (end -1.33 16.57) (stroke (width 0.12) (type solid)) (layer "F.SilkS"))
  (fp_line (start -1.33 16.57) (end 1.33 16.57) (stroke (width 0.12) (type solid)) (layer "F.SilkS"))
  (pad "1" thru_hole rect (at 0 0 90) (size 1.7 1.7) (drill 1) (layers "*.Cu" "*.Mask") (remove_unused_layers no) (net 6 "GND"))
  (pad "2" thru_hole oval (at 0 2.54 90) (size 1.7 1.7) (drill 1) (layers "*.Cu" "*.Mask") (remove_unused_layers no) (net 5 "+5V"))
  (pad "3" thru_hole oval (at 0 5.08 90) (size 1.7 1.7) (drill 1) (layers "*.Cu" "*.Mask") (remove_unused_layers no) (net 8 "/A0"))
  (pad "4" thru_hole oval (at 0 7.62 90) (size 1.7 1.7) (drill 1) (layers "*.Cu" "*.Mask") (remove_unused_layers no) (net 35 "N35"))
  (pad "5" thru_hole oval (at 0 10.16 90) (size 1.7 1.7) (drill 1) (layers "*.Cu" "*.Mask") (remove_unused_layers no) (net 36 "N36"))
  (pad "6" thru_hole oval (at 0 12.7 90) (size 1.7 1.7) (drill 1) (layers "*.Cu" "*.Mask") (remove_unused_layers no) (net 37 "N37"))
  (pad "7" thru_hole oval (at 0 15.24 90) (size 1.7 1.7) (drill 1) (layers "*.Cu" "*.Mask") (remove_unused_layers no) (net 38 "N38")))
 (gr_line (start 166.04 59.36) (end 168.58 61.9) (stroke (width 0.15) (type solid)) (layer "Edge.Cuts"))
 (gr_line (start 100 99.238) (end 100 47.422) (stroke (width 0.15) (type solid)) (layer "Edge.Cuts"))
 (gr_line (start 168.58 61.9) (end 168.58 96.19) (stroke (width 0.15) (type solid)) (layer "Edge.Cuts"))
 (gr_line (start 165.278 100) (end 100.762 100) (stroke (width 0.15) (type solid)) (layer "Edge.Cuts"))
 (gr_line (start 100.762 46.66) (end 163.5 46.66) (stroke (width 0.15) (type solid)) (layer "Edge.Cuts"))
 (gr_arc (start 100.762 100) (mid 100.223185 99.776815) (end 100 99.238) (stroke (width 0.15) (type solid)) (layer "Edge.Cuts"))
 (gr_line (start 168.58 96.19) (end 166.04 98.73) (stroke (width 0.15) (type solid)) (layer "Edge.Cuts"))
 (gr_line (start 163.5 46.66) (end 166.04 49.2) (stroke (width 0.15) (type solid)) (layer "Edge.Cuts"))
 (gr_arc (start 166.04 99.238) (mid 165.816815 99.776815) (end 165.278 100) (stroke (width 0.15) (type solid)) (layer "Edge.Cuts"))
 (gr_line (start 166.04 49.2) (end 166.04 59.36) (stroke (width 0.15) (type solid)) (layer "Edge.Cuts"))
 (gr_line (start 166.04 98.73) (end 166.04 99.238) (stroke (width 0.15) (type solid)) (layer "Edge.Cuts"))
 (gr_arc (start 100 47.422) (mid 100.223185 46.883185) (end 100.762 46.66) (stroke (width 0.15) (type solid)) (layer "Edge.Cuts"))
 (segment (start 146.92 93.5) (end 143.3 93.5) (width 1) (layer "F.Cu") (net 6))
 (segment (start 146.92 93.5) (end 147 93.5) (width 0.25) (layer "F.Cu") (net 6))
 (segment (start 138.182081 93.8) (end 120.6 93.8) (width 1) (layer "F.Cu") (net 6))
 (segment (start 117.2 82.7) (end 105.8 82.7) (width 1) (layer "F.Cu") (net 6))
 (segment (start 143.3 93.5) (end 140.64 96.16) (width 1) (layer "F.Cu") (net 6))
 (segment (start 147 93.5) (end 147 93.64) (width 0.25) (layer "F.Cu") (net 6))
 (segment (start 140.64 97.46) (end 140.64 96.257919) (width 1) (layer "F.Cu") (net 6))
 (segment (start 117.2 90.4) (end 117.2 82.7) (width 1) (layer "F.Cu") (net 6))
 (segment (start 120.6 93.8) (end 117.2 90.4) (width 1) (layer "F.Cu") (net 6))
 (segment (start 140.64 96.16) (end 140.64 97.46) (width 1) (layer "F.Cu") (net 6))
 (segment (start 140.64 96.257919) (end 138.182081 93.8) (width 1) (layer "F.Cu") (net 6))
 (segment (start 148.291469 95.708531) (end 149.46 94.54) (width 1) (layer "F.Cu") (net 5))
 (segment (start 138.1 97.46) (end 138.04 97.46) (width 0.25) (layer "F.Cu") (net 5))
 (segment (start 147.379874 99.4) (end 148.291469 98.488405) (width 1) (layer "F.Cu") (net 5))
 (segment (start 138.04 97.46) (end 138 97.5) (width 0.25) (layer "F.Cu") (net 5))
 (segment (start 149.46 94.54) (end 149.46 93.5) (width 1) (layer "F.Cu") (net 5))
 (segment (start 139.2 99.4) (end 147.379874 99.4) (width 1) (layer "F.Cu") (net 5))
 (segment (start 138.1 98.3) (end 139.2 99.4) (width 1) (layer "F.Cu") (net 5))
 (segment (start 138.1 97.46) (end 138.1 98.3) (width 1) (layer "F.Cu") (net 5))
 (segment (start 148.291469 98.488405) (end 148.291469 95.708531) (width 1) (layer "F.Cu") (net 5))
 (segment (start 150.8 97.46) (end 150.8 95.61) (width 1) (layer "F.Cu") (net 8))
 (segment (start 150.8 95.61) (end 152 94.41) (width 1) (layer "F.Cu") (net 8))
 (segment (start 152 94.41) (end 152 93.5) (width 1) (layer "F.Cu") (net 8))
 (segment (start 125.192103 52.807898) (end 126.323473 52.807898) (width 1) (layer "F.Cu") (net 15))
 (segment (start 128.956 50.175371) (end 128.956 49.2) (width 1) (layer "F.Cu") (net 15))
 (segment (start 126.323473 52.807898) (end 128.956 50.175371) (width 1) (layer "F.Cu") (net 15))
 (segment (start 131.6 50.2) (end 131.496 50.096) (width 1) (layer "F.Cu") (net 16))
 (segment (start 131.496 50.096) (end 131.496 49.2) (width 1) (layer "F.Cu") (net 16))
 (segment (start 124.6 89.6) (end 124.6 57.2) (width 1) (layer "F.Cu") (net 16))
 (segment (start 124.6 57.2) (end 131.6 50.2) (width 1) (layer "F.Cu") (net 16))
 (segment (start 146.36 79.64) (end 146.36 85.44) (width 1) (layer "F.Cu") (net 16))
 (segment (start 146.36 85.44) (end 142.2 89.6) (width 1) (layer "F.Cu") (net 16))
 (segment (start 142.2 89.6) (end 124.6 89.6) (width 1) (layer "F.Cu") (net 16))
 (segment (start 132.8 59.8) (end 140.4 52.2) (width 1) (layer "F.Cu") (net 20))
 (segment (start 141.656 50.744) (end 141.656 49.2) (width 1) (layer "F.Cu") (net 20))
 (segment (start 140.4 52.2) (end 140.4 52) (width 1) (layer "F.Cu") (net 20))
 (segment (start 132.8 65.6) (end 132.8 59.8) (width 1) (layer "F.Cu") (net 20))
 (segment (start 140.4 52) (end 141.656 50.744) (width 1) (layer "F.Cu") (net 20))
 (segment (start 136.04 79.64) (end 136.2 79.64) (width 1) (layer "F.Cu") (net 20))
 (segment (start 136.2 69) (end 132.8 65.6) (width 1) (layer "F.Cu") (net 20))
 (segment (start 136.04 79.64) (end 136 79.6) (width 1) (layer "F.Cu") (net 20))
 (segment (start 136.2 79.64) (end 136.2 69) (width 1) (layer "F.Cu") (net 20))
 (segment (start 142.592103 53.607898) (end 142.592103 52.327897) (width 1) (layer "F.Cu") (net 21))
 (segment (start 142.592103 52.327897) (end 145.72 49.2) (width 1) (layer "F.Cu") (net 21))
 (segment (start 126.6 57.8) (end 134.036 50.364) (width 1) (layer "F.Cu") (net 17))
 (segment (start 134.036 50.364) (end 134.036 49.2) (width 1) (layer "F.Cu") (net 17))
 (segment (start 139.8 87.8) (end 126.6 87.8) (width 1) (layer "F.Cu") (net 17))
 (segment (start 143.82 79.64) (end 143.82 83.78) (width 1) (layer "F.Cu") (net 17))
 (segment (start 126.6 87.8) (end 126.6 57.8) (width 1) (layer "F.Cu") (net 17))
 (segment (start 143.82 83.78) (end 139.8 87.8) (width 1) (layer "F.Cu") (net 17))
 (segment (start 136.576 50.424) (end 136.576 49.2) (width 1) (layer "F.Cu") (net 18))
 (segment (start 141.28 79.64) (end 141.28 82.32) (width 1) (layer "F.Cu") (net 18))
 (segment (start 128.6 83.8) (end 128.6 58.4) (width 1) (layer "F.Cu") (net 18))
 (segment (start 128.6 58.4) (end 136.576 50.424) (width 1) (layer "F.Cu") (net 18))
 (segment (start 130.6 85.8) (end 128.6 83.8) (width 1) (layer "F.Cu") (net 18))
 (segment (start 137.8 85.8) (end 130.6 85.8) (width 1) (layer "F.Cu") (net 18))
 (segment (start 141.28 82.32) (end 137.8 85.8) (width 1) (layer "F.Cu") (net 18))
 (segment (start 132.8 71) (end 130.4 68.6) (width 1) (layer "F.Cu") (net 19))
 (segment (start 132.8 83) (end 132.8 71) (width 1) (layer "F.Cu") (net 19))
 (segment (start 133 83.2) (end 132.8 83) (width 1) (layer "F.Cu") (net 19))
 (segment (start 139.116 50.884) (end 139.116 49.2) (width 1) (layer "F.Cu") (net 19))
 (segment (start 138.74 81.66) (end 137.2 83.2) (width 1) (layer "F.Cu") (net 19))
 (segment (start 138.74 79.64) (end 138.74 81.66) (width 1) (layer "F.Cu") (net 19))
 (segment (start 130.4 59.6) (end 139.116 50.884) (width 1) (layer "F.Cu") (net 19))
 (segment (start 137.2 83.2) (end 133 83.2) (width 1) (layer "F.Cu") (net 19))
 (segment (start 130.4 68.6) (end 130.4 59.6) (width 1) (layer "F.Cu") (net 19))
 (segment (start 154.392103 52.807898) (end 153.34 51.755795) (width 1) (layer "F.Cu") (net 24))
 (segment (start 153.34 51.755795) (end 153.34 49.2) (width 1) (layer "F.Cu") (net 24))
 (segment (start 148.9 64.4) (end 165 64.4) (width 1) (layer "F.Cu") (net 26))
 (segment (start 165.4 60.2) (end 165.4 57.2) (width 1) (layer "F.Cu") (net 26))
 (segment (start 165 64.4) (end 167.3 62.1) (width 1) (layer "F.Cu") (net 26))
 (segment (start 165.4 57.2) (end 158.42 50.22) (width 1) (layer "F.Cu") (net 26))
 (segment (start 158.42 50.22) (end 158.42 49.2) (width 1) (layer "F.Cu") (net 26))
 (segment (start 167.3 62.1) (end 165.4 60.2) (width 1) (layer "F.Cu") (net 26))
 (segment (start 142.6 57.07868) (end 148.26 51.41868) (width 1) (layer "F.Cu") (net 22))
 (segment (start 138.74 63.26) (end 142.6 59.4) (width 1) (layer "F.Cu") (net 22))
 (segment (start 142.6 59.4) (end 142.6 57.07868) (width 1) (layer "F.Cu") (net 22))
 (segment (start 138.74 64.4) (end 138.74 63.26) (width 1) (layer "F.Cu") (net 22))
 (segment (start 148.26 51.41868) (end 148.26 49.2) (width 1) (layer "F.Cu") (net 22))
 (segment (start 150.8 51.8) (end 150.8 49.2) (width 1) (layer "F.Cu") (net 23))
 (segment (start 144.6 60) (end 144.6 58) (width 1) (layer "F.Cu") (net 23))
 (segment (start 141.28 64.4) (end 141.28 63.32) (width 1) (layer "F.Cu") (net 23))
 (segment (start 141.28 63.32) (end 144.6 60) (width 1) (layer "F.Cu") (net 23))
 (segment (start 141.28 64.4) (end 141.4 64.4) (width 1) (layer "F.Cu") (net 23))
 (segment (start 144.6 58) (end 150.8 51.8) (width 1) (layer "F.Cu") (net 23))
 (segment (start 155.88 50.68) (end 155.88 49.2) (width 1) (layer "F.Cu") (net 25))
 (segment (start 163.2 60.6) (end 163.2 58) (width 1) (layer "F.Cu") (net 25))
 (segment (start 163.2 58) (end 155.88 50.68) (width 1) (layer "F.Cu") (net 25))
 (segment (start 145.54 97.46) (end 145.5 97.5) (width 0.25) (layer "F.Cu") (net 7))
 (segment (start 145.72 97.46) (end 145.54 97.46) (width 0.25) (layer "F.Cu") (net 7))
 (segment (start 136.2 64.4) (end 136.2 61.584205) (width 1) (layer "F.Cu") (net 29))
 (segment (start 102.2 49.05) (end 102.25 49.05) (width 0.25) (layer "F.Cu") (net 29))
 (segment (start 136.2 61.584205) (end 135.407898 60.792103) (width 1) (layer "F.Cu") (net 29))
 (segment (start 151.44 62.2) (end 153.04 60.6) (width 1) (layer "F.Cu") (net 33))
 (segment (start 146.36 63.64) (end 147.8 62.2) (width 1) (layer "F.Cu") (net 33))
 (segment (start 147.8 62.2) (end 151.44 62.2) (width 1) (layer "F.Cu") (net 33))
 (segment (start 146.36 64.4) (end 146.36 63.64) (width 1) (layer "F.Cu") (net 33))
 (segment (start 147.207898 60.192102) (end 147.207898 59.992103) (width 1) (layer "F.Cu") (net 34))
 (segment (start 143.82 64.4) (end 143.82 63.58) (width 1) (layer "F.Cu") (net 34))
 (segment (start 143.82 63.58) (end 147.207898 60.192102) (width 1) (layer "F.Cu") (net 34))
 (segment (start 122.4 64) (end 120.4 62) (width 1) (layer "F.Cu") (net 32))
 (segment (start 120.4 62) (end 120.015795 62) (width 1) (layer "F.Cu") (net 32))
 (segment (start 148.9 85.7) (end 143 91.6) (width 1) (layer "F.Cu") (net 32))
 (segment (start 143 91.6) (end 122.4 91.6) (width 1) (layer "F.Cu") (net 32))
 (segment (start 122.4 91.6) (end 122.4 64) (width 1) (layer "F.Cu") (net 32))
 (segment (start 120.015795 62) (end 118.007898 59.992103) (width 1) (layer "F.Cu") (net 32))
 (segment (start 148.9 79.64) (end 148.9 85.7) (width 1) (layer "F.Cu") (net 32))
 (segment (start 116.71066 78.2) (end 102.3 78.2) (width 1) (layer "F.Cu") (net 31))
 (segment (start 119.8 81.28934) (end 116.71066 78.2) (width 1) (layer "F.Cu") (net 31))
 (segment (start 119.8 87.6) (end 119.8 81.28934) (width 1) (layer "F.Cu") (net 31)))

